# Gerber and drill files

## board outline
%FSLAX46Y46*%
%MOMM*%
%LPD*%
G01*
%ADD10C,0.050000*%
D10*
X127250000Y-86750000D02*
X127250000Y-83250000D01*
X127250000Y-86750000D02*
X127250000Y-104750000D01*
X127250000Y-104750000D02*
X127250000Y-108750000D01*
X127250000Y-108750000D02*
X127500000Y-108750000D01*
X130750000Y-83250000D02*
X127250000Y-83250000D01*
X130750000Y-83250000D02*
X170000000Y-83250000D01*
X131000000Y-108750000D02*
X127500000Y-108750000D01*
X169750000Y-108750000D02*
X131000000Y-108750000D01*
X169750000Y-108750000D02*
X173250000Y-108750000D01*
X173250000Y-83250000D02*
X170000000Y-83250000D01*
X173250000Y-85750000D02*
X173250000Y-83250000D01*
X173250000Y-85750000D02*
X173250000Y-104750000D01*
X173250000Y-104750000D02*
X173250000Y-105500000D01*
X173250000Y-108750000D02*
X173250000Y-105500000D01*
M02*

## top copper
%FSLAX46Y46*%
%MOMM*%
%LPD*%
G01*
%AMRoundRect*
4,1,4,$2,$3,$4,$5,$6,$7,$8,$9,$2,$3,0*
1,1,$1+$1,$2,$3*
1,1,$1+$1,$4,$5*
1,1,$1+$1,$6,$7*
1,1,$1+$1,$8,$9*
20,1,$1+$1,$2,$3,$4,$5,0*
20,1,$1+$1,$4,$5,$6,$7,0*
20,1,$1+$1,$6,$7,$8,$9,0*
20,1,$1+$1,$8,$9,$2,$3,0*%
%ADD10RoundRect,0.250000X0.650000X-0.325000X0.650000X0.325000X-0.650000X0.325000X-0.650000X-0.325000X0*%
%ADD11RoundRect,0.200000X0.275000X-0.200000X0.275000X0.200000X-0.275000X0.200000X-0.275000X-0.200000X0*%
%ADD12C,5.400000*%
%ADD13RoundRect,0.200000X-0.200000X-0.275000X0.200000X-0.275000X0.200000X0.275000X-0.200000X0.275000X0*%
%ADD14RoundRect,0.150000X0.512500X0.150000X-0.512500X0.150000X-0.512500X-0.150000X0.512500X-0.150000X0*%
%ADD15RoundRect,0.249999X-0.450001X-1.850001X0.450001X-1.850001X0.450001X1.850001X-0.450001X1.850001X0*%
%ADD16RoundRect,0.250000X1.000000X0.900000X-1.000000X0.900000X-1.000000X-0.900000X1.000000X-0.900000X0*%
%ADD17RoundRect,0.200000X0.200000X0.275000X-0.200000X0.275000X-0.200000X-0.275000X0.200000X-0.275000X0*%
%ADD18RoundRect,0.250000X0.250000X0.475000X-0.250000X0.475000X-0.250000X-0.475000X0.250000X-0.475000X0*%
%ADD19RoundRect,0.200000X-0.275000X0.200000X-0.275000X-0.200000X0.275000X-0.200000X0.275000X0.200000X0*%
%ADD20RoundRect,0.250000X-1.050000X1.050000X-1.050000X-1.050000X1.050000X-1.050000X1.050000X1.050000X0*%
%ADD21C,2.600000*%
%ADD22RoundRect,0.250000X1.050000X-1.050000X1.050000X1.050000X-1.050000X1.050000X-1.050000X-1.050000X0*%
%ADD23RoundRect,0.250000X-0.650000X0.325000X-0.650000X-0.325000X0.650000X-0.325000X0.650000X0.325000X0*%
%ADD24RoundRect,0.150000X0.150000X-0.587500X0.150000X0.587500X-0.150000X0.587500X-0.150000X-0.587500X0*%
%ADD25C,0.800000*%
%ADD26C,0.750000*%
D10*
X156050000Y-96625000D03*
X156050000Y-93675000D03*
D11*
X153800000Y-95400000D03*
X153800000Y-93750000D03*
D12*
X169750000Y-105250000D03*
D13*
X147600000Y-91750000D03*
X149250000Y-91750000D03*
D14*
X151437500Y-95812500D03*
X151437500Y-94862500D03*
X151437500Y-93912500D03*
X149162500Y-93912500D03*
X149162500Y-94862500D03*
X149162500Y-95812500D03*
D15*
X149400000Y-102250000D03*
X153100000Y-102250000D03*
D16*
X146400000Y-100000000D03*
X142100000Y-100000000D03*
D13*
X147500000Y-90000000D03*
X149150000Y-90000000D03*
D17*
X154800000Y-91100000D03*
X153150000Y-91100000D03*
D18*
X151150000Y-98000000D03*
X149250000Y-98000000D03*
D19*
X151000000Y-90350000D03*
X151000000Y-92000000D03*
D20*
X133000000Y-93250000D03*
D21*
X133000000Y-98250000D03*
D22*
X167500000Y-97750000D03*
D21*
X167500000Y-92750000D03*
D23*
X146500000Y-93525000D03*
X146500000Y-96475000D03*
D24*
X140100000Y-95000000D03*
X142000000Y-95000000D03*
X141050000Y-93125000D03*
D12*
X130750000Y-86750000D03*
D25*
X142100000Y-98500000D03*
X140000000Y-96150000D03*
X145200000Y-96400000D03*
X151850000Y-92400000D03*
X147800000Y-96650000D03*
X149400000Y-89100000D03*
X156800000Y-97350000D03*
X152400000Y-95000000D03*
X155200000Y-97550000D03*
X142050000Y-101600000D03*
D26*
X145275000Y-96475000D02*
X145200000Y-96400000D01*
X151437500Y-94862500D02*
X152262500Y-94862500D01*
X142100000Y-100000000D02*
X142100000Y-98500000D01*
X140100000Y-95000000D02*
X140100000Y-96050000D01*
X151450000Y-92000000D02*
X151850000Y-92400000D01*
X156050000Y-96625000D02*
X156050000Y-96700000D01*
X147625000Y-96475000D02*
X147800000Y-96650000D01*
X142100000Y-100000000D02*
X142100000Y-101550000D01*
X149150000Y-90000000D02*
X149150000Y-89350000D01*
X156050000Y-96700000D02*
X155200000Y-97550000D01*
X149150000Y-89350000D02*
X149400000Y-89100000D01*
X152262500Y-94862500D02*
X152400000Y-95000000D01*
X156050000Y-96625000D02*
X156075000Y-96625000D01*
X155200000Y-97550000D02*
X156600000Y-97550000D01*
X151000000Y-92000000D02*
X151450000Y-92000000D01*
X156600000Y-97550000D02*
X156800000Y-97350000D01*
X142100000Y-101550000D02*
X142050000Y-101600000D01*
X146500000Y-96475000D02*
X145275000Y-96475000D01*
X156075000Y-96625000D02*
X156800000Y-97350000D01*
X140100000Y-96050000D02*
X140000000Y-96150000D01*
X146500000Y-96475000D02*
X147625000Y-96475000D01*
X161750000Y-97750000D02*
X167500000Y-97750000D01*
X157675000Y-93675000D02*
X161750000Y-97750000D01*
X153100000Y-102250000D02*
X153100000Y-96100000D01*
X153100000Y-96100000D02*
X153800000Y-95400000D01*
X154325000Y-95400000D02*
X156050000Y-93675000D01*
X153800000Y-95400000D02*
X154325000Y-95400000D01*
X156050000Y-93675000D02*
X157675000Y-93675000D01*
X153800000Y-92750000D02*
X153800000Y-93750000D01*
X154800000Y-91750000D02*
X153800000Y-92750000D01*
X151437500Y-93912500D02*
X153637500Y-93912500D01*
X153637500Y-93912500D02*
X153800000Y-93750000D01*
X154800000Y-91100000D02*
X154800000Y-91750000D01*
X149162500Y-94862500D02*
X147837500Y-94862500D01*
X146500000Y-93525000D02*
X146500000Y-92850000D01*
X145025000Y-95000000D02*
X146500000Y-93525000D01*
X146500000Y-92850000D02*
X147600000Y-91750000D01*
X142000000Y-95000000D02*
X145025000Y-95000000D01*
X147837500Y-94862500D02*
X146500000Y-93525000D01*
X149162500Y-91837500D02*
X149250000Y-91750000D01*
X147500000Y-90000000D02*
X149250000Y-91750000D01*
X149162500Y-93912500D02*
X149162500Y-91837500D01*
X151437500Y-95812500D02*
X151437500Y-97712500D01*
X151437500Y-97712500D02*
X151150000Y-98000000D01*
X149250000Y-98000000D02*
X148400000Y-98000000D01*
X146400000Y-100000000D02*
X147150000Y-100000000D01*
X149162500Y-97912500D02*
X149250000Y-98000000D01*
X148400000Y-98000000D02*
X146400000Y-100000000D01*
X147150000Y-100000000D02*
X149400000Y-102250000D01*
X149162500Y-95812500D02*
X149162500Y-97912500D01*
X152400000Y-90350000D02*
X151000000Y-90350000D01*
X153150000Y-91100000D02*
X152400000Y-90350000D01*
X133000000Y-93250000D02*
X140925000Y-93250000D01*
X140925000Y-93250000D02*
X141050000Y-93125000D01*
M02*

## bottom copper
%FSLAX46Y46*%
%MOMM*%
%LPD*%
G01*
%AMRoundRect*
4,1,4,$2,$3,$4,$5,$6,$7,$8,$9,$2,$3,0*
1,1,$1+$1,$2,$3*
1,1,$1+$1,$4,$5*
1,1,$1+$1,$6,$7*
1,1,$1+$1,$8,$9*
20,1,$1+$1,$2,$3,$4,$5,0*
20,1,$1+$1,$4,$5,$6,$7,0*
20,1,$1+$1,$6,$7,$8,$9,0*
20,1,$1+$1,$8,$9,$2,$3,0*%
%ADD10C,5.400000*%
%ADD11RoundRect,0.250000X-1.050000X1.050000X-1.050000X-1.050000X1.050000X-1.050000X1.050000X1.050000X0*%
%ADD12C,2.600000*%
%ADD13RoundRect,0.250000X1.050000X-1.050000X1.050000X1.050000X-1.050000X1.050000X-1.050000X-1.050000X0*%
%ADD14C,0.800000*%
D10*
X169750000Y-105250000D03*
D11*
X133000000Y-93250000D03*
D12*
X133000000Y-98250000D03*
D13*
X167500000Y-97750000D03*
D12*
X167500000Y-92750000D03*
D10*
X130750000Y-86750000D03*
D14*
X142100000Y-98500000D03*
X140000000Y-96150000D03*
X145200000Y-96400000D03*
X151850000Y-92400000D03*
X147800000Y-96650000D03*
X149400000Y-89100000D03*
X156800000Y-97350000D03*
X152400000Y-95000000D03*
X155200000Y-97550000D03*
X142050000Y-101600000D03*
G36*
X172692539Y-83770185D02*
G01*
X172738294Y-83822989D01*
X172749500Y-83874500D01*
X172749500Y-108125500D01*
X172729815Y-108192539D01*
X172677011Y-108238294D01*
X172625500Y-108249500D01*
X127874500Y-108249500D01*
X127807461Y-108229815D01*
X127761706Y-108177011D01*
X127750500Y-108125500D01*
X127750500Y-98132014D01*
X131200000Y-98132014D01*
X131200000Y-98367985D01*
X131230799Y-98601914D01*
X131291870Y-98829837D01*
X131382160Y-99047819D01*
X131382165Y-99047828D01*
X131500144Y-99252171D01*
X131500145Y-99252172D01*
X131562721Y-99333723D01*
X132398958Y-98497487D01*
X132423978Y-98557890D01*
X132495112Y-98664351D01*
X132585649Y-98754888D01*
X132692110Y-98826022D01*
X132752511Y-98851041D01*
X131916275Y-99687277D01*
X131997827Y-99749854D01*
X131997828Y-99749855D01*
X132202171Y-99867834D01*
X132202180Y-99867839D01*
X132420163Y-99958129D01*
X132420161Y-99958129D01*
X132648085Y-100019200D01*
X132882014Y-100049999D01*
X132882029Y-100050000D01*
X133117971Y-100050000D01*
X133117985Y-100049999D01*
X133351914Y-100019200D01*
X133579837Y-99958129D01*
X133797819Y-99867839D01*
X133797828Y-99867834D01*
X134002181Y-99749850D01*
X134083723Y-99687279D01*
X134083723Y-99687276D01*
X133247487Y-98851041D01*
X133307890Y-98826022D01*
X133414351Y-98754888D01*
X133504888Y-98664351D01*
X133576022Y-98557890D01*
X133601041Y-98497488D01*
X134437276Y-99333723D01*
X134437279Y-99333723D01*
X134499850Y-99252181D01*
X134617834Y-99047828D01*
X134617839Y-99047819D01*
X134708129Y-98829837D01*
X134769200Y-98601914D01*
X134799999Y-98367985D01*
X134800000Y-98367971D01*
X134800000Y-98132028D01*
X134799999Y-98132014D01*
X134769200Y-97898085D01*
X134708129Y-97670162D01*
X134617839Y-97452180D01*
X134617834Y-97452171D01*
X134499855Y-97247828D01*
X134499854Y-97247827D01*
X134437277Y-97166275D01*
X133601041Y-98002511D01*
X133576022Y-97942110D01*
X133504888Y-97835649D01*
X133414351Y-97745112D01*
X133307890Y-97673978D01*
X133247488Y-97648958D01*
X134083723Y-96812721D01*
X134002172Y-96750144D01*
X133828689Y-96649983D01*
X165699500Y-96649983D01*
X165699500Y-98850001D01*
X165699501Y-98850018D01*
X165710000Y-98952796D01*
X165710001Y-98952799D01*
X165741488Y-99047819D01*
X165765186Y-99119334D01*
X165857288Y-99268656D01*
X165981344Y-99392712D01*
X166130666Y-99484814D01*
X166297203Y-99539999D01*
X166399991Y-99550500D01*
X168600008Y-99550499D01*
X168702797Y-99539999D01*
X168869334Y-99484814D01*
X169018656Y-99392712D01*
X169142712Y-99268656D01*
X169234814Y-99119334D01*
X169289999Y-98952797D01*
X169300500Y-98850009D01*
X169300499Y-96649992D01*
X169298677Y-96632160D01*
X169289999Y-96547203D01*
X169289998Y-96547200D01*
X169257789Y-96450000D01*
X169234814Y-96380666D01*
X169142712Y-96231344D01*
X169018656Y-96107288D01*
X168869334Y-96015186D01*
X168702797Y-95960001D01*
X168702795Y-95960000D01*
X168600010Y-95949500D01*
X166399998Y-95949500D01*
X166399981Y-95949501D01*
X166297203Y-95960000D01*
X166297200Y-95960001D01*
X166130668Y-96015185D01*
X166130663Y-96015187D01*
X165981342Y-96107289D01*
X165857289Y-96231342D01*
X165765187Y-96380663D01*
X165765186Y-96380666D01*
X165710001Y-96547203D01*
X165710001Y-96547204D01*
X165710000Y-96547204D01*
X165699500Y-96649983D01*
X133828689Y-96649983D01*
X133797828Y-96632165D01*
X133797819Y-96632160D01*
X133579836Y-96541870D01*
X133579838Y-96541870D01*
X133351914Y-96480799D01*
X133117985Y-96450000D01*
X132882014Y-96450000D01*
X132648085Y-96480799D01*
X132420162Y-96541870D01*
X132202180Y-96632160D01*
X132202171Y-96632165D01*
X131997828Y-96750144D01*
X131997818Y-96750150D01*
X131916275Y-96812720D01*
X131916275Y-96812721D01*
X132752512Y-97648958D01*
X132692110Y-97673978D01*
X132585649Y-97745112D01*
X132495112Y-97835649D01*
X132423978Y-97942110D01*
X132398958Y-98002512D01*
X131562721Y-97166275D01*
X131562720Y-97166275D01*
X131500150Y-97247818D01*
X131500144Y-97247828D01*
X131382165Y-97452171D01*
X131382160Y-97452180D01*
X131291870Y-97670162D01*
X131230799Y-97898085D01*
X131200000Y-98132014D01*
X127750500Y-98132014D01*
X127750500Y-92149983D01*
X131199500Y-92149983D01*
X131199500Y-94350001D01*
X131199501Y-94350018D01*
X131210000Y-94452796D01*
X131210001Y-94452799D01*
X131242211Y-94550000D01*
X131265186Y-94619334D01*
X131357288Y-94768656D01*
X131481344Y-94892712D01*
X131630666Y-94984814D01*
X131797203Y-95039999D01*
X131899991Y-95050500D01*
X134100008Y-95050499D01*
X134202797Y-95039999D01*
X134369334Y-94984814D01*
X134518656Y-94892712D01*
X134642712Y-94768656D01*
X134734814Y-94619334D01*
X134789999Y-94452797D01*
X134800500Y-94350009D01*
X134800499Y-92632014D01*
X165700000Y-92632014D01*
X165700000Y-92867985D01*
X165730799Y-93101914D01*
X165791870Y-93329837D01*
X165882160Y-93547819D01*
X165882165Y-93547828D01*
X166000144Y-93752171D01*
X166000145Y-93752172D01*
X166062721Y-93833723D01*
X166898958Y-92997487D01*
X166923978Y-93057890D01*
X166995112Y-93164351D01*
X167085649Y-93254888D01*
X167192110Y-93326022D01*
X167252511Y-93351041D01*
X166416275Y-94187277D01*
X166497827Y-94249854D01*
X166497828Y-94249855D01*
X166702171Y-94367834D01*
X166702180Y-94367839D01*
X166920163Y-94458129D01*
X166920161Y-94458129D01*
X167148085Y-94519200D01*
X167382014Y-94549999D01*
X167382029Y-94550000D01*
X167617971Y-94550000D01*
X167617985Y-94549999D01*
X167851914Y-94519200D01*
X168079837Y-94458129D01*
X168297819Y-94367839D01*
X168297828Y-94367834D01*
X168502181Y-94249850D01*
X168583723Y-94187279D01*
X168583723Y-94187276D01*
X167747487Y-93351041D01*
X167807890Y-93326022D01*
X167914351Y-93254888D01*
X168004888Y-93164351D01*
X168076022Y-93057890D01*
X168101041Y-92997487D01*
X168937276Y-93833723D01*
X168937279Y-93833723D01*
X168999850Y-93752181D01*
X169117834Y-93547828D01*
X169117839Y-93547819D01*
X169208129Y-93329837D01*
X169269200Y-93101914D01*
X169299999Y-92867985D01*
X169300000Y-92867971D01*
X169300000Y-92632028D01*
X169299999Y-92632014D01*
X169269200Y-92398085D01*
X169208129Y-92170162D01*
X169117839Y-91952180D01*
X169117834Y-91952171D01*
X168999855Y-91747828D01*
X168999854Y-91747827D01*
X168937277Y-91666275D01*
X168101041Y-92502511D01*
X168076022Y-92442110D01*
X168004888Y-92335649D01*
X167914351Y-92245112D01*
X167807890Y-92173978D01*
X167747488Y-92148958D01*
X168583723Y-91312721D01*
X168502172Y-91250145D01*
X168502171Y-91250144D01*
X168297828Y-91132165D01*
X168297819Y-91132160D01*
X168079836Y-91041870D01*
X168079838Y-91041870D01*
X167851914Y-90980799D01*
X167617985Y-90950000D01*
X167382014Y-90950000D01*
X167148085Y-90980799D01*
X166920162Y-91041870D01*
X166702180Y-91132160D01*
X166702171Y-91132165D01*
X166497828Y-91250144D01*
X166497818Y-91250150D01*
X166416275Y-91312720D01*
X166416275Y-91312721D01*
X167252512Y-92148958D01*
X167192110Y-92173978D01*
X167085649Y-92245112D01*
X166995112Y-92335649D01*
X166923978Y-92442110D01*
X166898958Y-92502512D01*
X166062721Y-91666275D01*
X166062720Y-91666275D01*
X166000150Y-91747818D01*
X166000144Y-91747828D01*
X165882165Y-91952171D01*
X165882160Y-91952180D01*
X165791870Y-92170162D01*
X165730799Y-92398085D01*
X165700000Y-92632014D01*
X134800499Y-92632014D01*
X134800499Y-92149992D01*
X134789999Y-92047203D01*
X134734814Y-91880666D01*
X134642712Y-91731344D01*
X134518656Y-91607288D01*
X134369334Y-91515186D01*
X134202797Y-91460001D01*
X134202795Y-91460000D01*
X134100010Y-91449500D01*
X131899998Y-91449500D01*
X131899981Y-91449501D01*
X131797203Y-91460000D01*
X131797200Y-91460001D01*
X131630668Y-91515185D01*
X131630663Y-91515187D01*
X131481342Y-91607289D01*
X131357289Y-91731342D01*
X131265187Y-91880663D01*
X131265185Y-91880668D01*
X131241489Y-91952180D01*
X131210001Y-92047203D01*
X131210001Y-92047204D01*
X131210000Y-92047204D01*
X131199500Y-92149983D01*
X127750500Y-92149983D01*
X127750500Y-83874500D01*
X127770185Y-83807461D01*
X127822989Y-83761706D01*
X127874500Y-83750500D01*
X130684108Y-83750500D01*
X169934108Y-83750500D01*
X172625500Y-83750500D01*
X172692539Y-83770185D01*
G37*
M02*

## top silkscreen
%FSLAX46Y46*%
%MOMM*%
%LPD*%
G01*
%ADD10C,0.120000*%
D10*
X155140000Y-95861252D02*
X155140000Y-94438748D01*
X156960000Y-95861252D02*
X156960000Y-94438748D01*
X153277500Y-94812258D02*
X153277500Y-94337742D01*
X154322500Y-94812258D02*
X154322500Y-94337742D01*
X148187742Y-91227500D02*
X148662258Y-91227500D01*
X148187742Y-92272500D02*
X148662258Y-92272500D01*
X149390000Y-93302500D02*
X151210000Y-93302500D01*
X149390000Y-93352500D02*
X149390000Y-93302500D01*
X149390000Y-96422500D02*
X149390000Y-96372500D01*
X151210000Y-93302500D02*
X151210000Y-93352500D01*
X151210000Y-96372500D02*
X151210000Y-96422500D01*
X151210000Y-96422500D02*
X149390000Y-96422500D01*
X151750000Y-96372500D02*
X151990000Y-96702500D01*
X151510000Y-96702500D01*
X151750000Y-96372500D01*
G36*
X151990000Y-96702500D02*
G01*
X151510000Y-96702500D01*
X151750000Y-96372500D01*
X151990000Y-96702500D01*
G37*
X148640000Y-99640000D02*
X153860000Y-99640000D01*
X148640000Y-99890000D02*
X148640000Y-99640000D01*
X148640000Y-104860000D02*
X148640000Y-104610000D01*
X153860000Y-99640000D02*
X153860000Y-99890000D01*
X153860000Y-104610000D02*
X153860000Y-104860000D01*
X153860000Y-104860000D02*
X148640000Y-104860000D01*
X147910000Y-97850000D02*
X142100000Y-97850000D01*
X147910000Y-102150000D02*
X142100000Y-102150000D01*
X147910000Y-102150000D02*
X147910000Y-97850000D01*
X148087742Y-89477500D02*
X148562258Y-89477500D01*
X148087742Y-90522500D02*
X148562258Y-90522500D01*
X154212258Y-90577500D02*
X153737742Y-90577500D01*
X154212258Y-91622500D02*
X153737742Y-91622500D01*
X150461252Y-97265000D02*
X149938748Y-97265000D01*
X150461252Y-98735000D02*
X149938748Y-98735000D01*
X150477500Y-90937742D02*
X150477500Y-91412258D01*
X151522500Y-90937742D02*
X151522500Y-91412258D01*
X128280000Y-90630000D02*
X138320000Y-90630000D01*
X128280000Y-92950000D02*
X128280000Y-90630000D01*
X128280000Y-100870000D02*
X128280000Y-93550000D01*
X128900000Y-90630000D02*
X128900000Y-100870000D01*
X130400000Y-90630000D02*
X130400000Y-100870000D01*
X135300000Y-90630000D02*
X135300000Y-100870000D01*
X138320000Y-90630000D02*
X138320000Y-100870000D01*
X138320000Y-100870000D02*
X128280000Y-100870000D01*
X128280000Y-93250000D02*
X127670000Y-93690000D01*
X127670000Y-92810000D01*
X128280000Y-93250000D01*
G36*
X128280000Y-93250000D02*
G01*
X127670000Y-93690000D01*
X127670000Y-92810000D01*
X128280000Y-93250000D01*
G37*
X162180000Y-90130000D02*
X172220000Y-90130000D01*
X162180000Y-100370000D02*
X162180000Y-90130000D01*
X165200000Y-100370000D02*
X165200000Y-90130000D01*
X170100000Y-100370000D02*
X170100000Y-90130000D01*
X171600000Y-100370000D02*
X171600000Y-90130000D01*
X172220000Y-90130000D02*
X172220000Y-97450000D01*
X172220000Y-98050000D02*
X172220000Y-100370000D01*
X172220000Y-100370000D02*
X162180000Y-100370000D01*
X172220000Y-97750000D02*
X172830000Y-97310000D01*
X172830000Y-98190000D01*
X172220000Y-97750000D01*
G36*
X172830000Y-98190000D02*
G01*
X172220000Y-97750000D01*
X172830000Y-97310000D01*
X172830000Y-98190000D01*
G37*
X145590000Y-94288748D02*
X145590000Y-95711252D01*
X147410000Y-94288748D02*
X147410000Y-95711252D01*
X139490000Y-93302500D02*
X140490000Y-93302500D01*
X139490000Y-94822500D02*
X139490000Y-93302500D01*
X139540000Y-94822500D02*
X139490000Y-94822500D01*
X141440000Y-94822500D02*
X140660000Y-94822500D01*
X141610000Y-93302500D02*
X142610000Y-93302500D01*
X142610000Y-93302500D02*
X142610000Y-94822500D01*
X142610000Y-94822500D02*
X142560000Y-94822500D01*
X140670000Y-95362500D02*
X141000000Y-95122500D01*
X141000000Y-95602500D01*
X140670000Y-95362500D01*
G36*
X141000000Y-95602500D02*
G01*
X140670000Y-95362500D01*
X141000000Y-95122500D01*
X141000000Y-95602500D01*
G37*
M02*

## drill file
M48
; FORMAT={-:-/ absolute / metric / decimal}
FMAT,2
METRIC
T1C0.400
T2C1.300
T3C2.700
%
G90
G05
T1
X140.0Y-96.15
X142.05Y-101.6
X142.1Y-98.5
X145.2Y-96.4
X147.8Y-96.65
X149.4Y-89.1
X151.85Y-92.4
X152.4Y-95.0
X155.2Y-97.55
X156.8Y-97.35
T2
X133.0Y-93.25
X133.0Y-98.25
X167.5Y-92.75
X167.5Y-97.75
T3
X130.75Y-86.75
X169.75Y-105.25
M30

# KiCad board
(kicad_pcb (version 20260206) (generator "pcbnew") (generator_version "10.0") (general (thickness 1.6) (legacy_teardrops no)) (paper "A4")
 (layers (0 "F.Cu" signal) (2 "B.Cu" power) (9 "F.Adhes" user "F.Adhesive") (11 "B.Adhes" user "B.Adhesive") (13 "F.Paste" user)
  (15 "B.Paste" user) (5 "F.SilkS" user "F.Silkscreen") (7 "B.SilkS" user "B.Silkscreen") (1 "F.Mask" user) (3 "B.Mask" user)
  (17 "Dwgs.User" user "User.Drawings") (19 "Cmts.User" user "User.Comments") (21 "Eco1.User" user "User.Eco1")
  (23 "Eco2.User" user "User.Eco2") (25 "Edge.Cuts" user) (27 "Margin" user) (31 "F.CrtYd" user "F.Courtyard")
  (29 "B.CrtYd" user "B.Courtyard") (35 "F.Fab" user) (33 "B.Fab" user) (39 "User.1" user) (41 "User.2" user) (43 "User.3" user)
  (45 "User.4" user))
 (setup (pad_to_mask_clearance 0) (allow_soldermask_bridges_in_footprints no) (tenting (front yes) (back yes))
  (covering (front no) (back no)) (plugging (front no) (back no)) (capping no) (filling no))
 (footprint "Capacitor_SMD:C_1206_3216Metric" (layer "F.Cu") (at 156.05 95.15 90)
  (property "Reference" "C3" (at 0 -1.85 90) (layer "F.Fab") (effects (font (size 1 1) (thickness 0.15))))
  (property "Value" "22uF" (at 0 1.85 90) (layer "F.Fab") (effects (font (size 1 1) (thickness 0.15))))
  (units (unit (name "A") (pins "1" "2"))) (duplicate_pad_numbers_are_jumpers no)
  (fp_line (start -0.711252 -0.91) (end 0.711252 -0.91) (stroke (width 0.12) (type solid)) (layer "F.SilkS"))
  (fp_line (start -0.711252 0.91) (end 0.711252 0.91) (stroke (width 0.12) (type solid)) (layer "F.SilkS"))
  (pad "1" smd roundrect (at -1.475 0 90) (size 1.15 1.8) (layers "F.Cu" "F.Mask" "F.Paste") (roundrect_rratio 0.217391) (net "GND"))
  (pad "2" smd roundrect (at 1.475 0 90) (size 1.15 1.8) (layers "F.Cu" "F.Mask" "F.Paste") (roundrect_rratio 0.217391) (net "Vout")))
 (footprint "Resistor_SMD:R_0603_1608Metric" (layer "F.Cu") (at 153.8 94.575 90)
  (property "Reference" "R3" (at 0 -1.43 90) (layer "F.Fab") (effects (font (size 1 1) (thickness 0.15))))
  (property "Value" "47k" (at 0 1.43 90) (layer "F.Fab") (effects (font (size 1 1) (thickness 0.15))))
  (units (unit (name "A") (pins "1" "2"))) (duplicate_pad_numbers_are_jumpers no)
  (fp_line (start -0.237258 -0.5225) (end 0.237258 -0.5225) (stroke (width 0.12) (type solid)) (layer "F.SilkS"))
  (fp_line (start -0.237258 0.5225) (end 0.237258 0.5225) (stroke (width 0.12) (type solid)) (layer "F.SilkS"))
  (pad "1" smd roundrect (at -0.825 0 90) (size 0.8 0.95) (layers "F.Cu" "F.Mask" "F.Paste") (roundrect_rratio 0.25) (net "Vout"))
  (pad "2" smd roundrect (at 0.825 0 90) (size 0.8 0.95) (layers "F.Cu" "F.Mask" "F.Paste") (roundrect_rratio 0.25) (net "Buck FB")))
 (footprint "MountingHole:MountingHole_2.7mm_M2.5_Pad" (layer "F.Cu") (at 169.75 105.25)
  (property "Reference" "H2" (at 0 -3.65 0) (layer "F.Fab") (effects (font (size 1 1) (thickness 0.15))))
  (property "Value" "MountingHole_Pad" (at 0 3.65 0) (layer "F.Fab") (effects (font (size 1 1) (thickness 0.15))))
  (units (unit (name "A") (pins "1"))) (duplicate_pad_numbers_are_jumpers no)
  (pad "1" thru_hole circle (at 0 0) (size 5.4 5.4) (drill 2.7) (layers "*.Cu" "*.Mask") (remove_unused_layers no) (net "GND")
   (zone_connect 2)))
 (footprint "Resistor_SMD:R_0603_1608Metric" (layer "F.Cu") (at 148.425 91.75)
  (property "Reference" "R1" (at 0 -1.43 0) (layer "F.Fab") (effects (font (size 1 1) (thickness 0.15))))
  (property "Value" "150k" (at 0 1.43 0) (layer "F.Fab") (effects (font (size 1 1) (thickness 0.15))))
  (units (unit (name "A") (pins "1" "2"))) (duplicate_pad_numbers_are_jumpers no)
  (fp_line (start -0.237258 -0.5225) (end 0.237258 -0.5225) (stroke (width 0.12) (type solid)) (layer "F.SilkS"))
  (fp_line (start -0.237258 0.5225) (end 0.237258 0.5225) (stroke (width 0.12) (type solid)) (layer "F.SilkS"))
  (pad "1" smd roundrect (at -0.825 0) (size 0.8 0.95) (layers "F.Cu" "F.Mask" "F.Paste") (roundrect_rratio 0.25) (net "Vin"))
  (pad "2" smd roundrect (at 0.825 0) (size 0.8 0.95) (layers "F.Cu" "F.Mask" "F.Paste") (roundrect_rratio 0.25) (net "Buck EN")))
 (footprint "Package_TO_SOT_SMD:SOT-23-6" (layer "F.Cu") (at 150.3 94.8625 180)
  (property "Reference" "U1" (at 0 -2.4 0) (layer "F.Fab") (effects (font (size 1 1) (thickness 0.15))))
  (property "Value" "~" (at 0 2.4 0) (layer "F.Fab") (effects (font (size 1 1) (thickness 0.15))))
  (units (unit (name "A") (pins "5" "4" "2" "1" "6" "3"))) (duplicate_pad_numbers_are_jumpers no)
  (fp_line (start 0.91 1.56) (end -0.91 1.56) (stroke (width 0.12) (type solid)) (layer "F.SilkS"))
  (fp_line (start 0.91 1.51) (end 0.91 1.56) (stroke (width 0.12) (type solid)) (layer "F.SilkS"))
  (fp_line (start 0.91 -1.56) (end 0.91 -1.51) (stroke (width 0.12) (type solid)) (layer "F.SilkS"))
  (fp_line (start -0.91 1.56) (end -0.91 1.51) (stroke (width 0.12) (type solid)) (layer "F.SilkS"))
  (fp_line (start -0.91 -1.51) (end -0.91 -1.56) (stroke (width 0.12) (type solid)) (layer "F.SilkS"))
  (fp_line (start -0.91 -1.56) (end 0.91 -1.56) (stroke (width 0.12) (type solid)) (layer "F.SilkS"))
  (fp_poly (pts (xy -1.45 -1.51) (xy -1.69 -1.84) (xy -1.21 -1.84)) (stroke (width 0.12) (type solid)) (fill yes) (layer "F.SilkS"))
  (pad "1" smd roundrect (at -1.1375 -0.95 180) (size 1.325 0.6) (layers "F.Cu" "F.Mask" "F.Paste") (roundrect_rratio 0.25) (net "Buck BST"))
  (pad "2" smd roundrect (at -1.1375 0 180) (size 1.325 0.6) (layers "F.Cu" "F.Mask" "F.Paste") (roundrect_rratio 0.25) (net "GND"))
  (pad "3" smd roundrect (at -1.1375 0.95 180) (size 1.325 0.6) (layers "F.Cu" "F.Mask" "F.Paste") (roundrect_rratio 0.25) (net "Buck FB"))
  (pad "4" smd roundrect (at 1.1375 0.95 180) (size 1.325 0.6) (layers "F.Cu" "F.Mask" "F.Paste") (roundrect_rratio 0.25) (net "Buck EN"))
  (pad "5" smd roundrect (at 1.1375 0 180) (size 1.325 0.6) (layers "F.Cu" "F.Mask" "F.Paste") (roundrect_rratio 0.25) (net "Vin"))
  (pad "6" smd roundrect (at 1.1375 -0.95 180) (size 1.325 0.6) (layers "F.Cu" "F.Mask" "F.Paste") (roundrect_rratio 0.25) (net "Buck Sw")))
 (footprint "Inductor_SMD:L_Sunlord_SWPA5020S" (layer "F.Cu") (at 151.25 102.25)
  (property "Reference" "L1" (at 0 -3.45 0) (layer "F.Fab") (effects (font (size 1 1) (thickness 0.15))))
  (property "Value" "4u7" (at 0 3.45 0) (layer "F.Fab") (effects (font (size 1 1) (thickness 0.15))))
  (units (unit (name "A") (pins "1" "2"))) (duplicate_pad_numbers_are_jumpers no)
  (fp_line (start -2.61 -2.61) (end 2.61 -2.61) (stroke (width 0.12) (type solid)) (layer "F.SilkS"))
  (fp_line (start -2.61 -2.36) (end -2.61 -2.61) (stroke (width 0.12) (type solid)) (layer "F.SilkS"))
  (fp_line (start -2.61 2.61) (end -2.61 2.36) (stroke (width 0.12) (type solid)) (layer "F.SilkS"))
  (fp_line (start 2.61 -2.61) (end 2.61 -2.36) (stroke (width 0.12) (type solid)) (layer "F.SilkS"))
  (fp_line (start 2.61 2.36) (end 2.61 2.61) (stroke (width 0.12) (type solid)) (layer "F.SilkS"))
  (fp_line (start 2.61 2.61) (end -2.61 2.61) (stroke (width 0.12) (type solid)) (layer "F.SilkS"))
  (pad "1" smd roundrect (at -1.85 0) (size 1.4 4.2) (layers "F.Cu" "F.Mask" "F.Paste") (roundrect_rratio 0.178571) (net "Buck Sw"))
  (pad "2" smd roundrect (at 1.85 0) (size 1.4 4.2) (layers "F.Cu" "F.Mask" "F.Paste") (roundrect_rratio 0.178571) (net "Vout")))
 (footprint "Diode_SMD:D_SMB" (layer "F.Cu") (at 144.25 100 180)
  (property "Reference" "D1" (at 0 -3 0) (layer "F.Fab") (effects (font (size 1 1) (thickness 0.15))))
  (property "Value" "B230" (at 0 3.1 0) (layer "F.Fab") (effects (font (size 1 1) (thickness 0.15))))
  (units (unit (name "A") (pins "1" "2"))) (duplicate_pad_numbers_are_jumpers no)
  (fp_line (start -3.66 2.15) (end 2.15 2.15) (stroke (width 0.12) (type solid)) (layer "F.SilkS"))
  (fp_line (start -3.66 -2.15) (end 2.15 -2.15) (stroke (width 0.12) (type solid)) (layer "F.SilkS"))
  (fp_line (start -3.66 -2.15) (end -3.66 2.15) (stroke (width 0.12) (type solid)) (layer "F.SilkS"))
  (pad "1" smd roundrect (at -2.15 0 180) (size 2.5 2.3) (layers "F.Cu" "F.Mask" "F.Paste") (roundrect_rratio 0.1086956522) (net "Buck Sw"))
  (pad "2" smd roundrect (at 2.15 0 180) (size 2.5 2.3) (layers "F.Cu" "F.Mask" "F.Paste") (roundrect_rratio 0.1086956522) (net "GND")))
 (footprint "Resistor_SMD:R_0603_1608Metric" (layer "F.Cu") (at 148.325 90)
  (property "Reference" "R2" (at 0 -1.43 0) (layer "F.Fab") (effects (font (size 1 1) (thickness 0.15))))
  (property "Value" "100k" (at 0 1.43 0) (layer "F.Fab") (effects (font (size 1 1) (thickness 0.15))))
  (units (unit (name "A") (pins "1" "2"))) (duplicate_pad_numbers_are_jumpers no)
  (fp_line (start -0.237258 -0.5225) (end 0.237258 -0.5225) (stroke (width 0.12) (type solid)) (layer "F.SilkS"))
  (fp_line (start -0.237258 0.5225) (end 0.237258 0.5225) (stroke (width 0.12) (type solid)) (layer "F.SilkS"))
  (pad "1" smd roundrect (at -0.825 0) (size 0.8 0.95) (layers "F.Cu" "F.Mask" "F.Paste") (roundrect_rratio 0.25) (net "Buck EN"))
  (pad "2" smd roundrect (at 0.825 0) (size 0.8 0.95) (layers "F.Cu" "F.Mask" "F.Paste") (roundrect_rratio 0.25) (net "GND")))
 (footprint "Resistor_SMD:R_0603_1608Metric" (layer "F.Cu") (at 153.975 91.1 180)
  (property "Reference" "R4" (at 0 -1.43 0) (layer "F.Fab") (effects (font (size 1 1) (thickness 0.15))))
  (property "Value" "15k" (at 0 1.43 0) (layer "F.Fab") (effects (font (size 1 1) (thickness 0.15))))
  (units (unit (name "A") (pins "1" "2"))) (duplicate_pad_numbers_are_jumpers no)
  (fp_line (start -0.237258 0.5225) (end 0.237258 0.5225) (stroke (width 0.12) (type solid)) (layer "F.SilkS"))
  (fp_line (start -0.237258 -0.5225) (end 0.237258 -0.5225) (stroke (width 0.12) (type solid)) (layer "F.SilkS"))
  (pad "1" smd roundrect (at -0.825 0 180) (size 0.8 0.95) (layers "F.Cu" "F.Mask" "F.Paste") (roundrect_rratio 0.25) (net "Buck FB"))
  (pad "2" smd roundrect (at 0.825 0 180) (size 0.8 0.95) (layers "F.Cu" "F.Mask" "F.Paste") (roundrect_rratio 0.25) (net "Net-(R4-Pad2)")))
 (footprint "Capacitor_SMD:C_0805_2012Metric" (layer "F.Cu") (at 150.2 98 180)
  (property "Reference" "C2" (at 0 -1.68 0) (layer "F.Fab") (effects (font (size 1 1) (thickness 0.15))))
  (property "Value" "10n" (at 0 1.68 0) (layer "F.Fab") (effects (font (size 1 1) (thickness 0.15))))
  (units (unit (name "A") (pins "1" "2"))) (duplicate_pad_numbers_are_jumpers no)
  (fp_line (start -0.261252 0.735) (end 0.261252 0.735) (stroke (width 0.12) (type solid)) (layer "F.SilkS"))
  (fp_line (start -0.261252 -0.735) (end 0.261252 -0.735) (stroke (width 0.12) (type solid)) (layer "F.SilkS"))
  (pad "1" smd roundrect (at -0.95 0 180) (size 1 1.45) (layers "F.Cu" "F.Mask" "F.Paste") (roundrect_rratio 0.25) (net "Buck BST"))
  (pad "2" smd roundrect (at 0.95 0 180) (size 1 1.45) (layers "F.Cu" "F.Mask" "F.Paste") (roundrect_rratio 0.25) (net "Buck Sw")))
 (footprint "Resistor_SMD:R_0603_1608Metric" (layer "F.Cu") (at 151 91.175 -90)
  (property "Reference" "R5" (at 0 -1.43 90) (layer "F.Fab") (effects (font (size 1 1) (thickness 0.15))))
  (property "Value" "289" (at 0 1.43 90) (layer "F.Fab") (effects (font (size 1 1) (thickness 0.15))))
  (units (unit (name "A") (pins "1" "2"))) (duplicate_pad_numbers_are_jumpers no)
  (fp_line (start -0.237258 0.5225) (end 0.237258 0.5225) (stroke (width 0.12) (type solid)) (layer "F.SilkS"))
  (fp_line (start -0.237258 -0.5225) (end 0.237258 -0.5225) (stroke (width 0.12) (type solid)) (layer "F.SilkS"))
  (pad "1" smd roundrect (at -0.825 0 270) (size 0.8 0.95) (layers "F.Cu" "F.Mask" "F.Paste") (roundrect_rratio 0.25) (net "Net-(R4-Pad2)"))
  (pad "2" smd roundrect (at 0.825 0 270) (size 0.8 0.95) (layers "F.Cu" "F.Mask" "F.Paste") (roundrect_rratio 0.25) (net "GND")))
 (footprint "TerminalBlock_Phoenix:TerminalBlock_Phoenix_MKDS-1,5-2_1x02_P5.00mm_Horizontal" (layer "F.Cu") (at 133 93.25 -90)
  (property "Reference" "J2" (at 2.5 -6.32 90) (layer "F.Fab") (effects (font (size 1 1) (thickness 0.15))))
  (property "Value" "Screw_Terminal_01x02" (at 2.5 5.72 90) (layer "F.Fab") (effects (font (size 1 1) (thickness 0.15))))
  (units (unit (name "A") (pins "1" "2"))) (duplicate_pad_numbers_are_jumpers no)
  (fp_line (start -2.62 4.72) (end -2.62 -5.32) (stroke (width 0.12) (type solid)) (layer "F.SilkS"))
  (fp_line (start -0.3 4.72) (end -2.62 4.72) (stroke (width 0.12) (type solid)) (layer "F.SilkS"))
  (fp_line (start 7.62 4.72) (end 0.3 4.72) (stroke (width 0.12) (type solid)) (layer "F.SilkS"))
  (fp_line (start -2.62 4.1) (end 7.62 4.1) (stroke (width 0.12) (type solid)) (layer "F.SilkS"))
  (fp_line (start -2.62 2.6) (end 7.62 2.6) (stroke (width 0.12) (type solid)) (layer "F.SilkS"))
  (fp_line (start -2.62 -2.3) (end 7.62 -2.3) (stroke (width 0.12) (type solid)) (layer "F.SilkS"))
  (fp_line (start -2.62 -5.32) (end 7.62 -5.32) (stroke (width 0.12) (type solid)) (layer "F.SilkS"))
  (fp_line (start 7.62 -5.32) (end 7.62 4.72) (stroke (width 0.12) (type solid)) (layer "F.SilkS"))
  (fp_poly (pts (xy 0 4.72) (xy 0.44 5.33) (xy -0.44 5.33)) (stroke (width 0.12) (type solid)) (fill yes) (layer "F.SilkS"))
  (pad "1" thru_hole roundrect (at 0 0 270) (size 2.6 2.6) (drill 1.3) (layers "*.Cu" "*.Mask") (remove_unused_layers no)
   (roundrect_rratio 0.096154) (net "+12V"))
  (pad "2" thru_hole circle (at 5 0 270) (size 2.6 2.6) (drill 1.3) (layers "*.Cu" "*.Mask") (remove_unused_layers no) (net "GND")))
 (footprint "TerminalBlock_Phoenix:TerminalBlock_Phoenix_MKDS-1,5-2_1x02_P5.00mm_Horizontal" (layer "F.Cu") (at 167.5 97.75 90)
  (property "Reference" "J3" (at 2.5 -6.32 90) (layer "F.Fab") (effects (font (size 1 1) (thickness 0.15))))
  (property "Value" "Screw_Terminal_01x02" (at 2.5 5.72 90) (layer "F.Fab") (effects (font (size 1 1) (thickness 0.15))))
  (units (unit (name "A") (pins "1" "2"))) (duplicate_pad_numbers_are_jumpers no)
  (fp_line (start 7.62 -5.32) (end 7.62 4.72) (stroke (width 0.12) (type solid)) (layer "F.SilkS"))
  (fp_line (start -2.62 -5.32) (end 7.62 -5.32) (stroke (width 0.12) (type solid)) (layer "F.SilkS"))
  (fp_line (start -2.62 -2.3) (end 7.62 -2.3) (stroke (width 0.12) (type solid)) (layer "F.SilkS"))
  (fp_line (start -2.62 2.6) (end 7.62 2.6) (stroke (width 0.12) (type solid)) (layer "F.SilkS"))
  (fp_line (start -2.62 4.1) (end 7.62 4.1) (stroke (width 0.12) (type solid)) (layer "F.SilkS"))
  (fp_line (start 7.62 4.72) (end 0.3 4.72) (stroke (width 0.12) (type solid)) (layer "F.SilkS"))
  (fp_line (start -0.3 4.72) (end -2.62 4.72) (stroke (width 0.12) (type solid)) (layer "F.SilkS"))
  (fp_line (start -2.62 4.72) (end -2.62 -5.32) (stroke (width 0.12) (type solid)) (layer "F.SilkS"))
  (fp_poly (pts (xy 0 4.72) (xy 0.44 5.33) (xy -0.44 5.33)) (stroke (width 0.12) (type solid)) (fill yes) (layer "F.SilkS"))
  (pad "1" thru_hole roundrect (at 0 0 90) (size 2.6 2.6) (drill 1.3) (layers "*.Cu" "*.Mask") (remove_unused_layers no)
   (roundrect_rratio 0.096154) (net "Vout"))
  (pad "2" thru_hole circle (at 5 0 90) (size 2.6 2.6) (drill 1.3) (layers "*.Cu" "*.Mask") (remove_unused_layers no) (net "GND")))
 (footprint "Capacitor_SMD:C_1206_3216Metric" (layer "F.Cu") (at 146.5 95 -90)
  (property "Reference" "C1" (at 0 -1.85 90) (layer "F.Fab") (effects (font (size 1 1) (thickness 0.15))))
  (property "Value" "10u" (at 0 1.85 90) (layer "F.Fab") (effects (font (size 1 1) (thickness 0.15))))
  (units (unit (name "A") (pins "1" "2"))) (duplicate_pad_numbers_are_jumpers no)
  (fp_line (start -0.711252 0.91) (end 0.711252 0.91) (stroke (width 0.12) (type solid)) (layer "F.SilkS"))
  (fp_line (start -0.711252 -0.91) (end 0.711252 -0.91) (stroke (width 0.12) (type solid)) (layer "F.SilkS"))
  (pad "1" smd roundrect (at -1.475 0 270) (size 1.15 1.8) (layers "F.Cu" "F.Mask" "F.Paste") (roundrect_rratio 0.217391) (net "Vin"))
  (pad "2" smd roundrect (at 1.475 0 270) (size 1.15 1.8) (layers "F.Cu" "F.Mask" "F.Paste") (roundrect_rratio 0.217391) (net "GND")))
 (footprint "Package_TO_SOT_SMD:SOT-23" (layer "F.Cu") (at 141.05 94.0625 90)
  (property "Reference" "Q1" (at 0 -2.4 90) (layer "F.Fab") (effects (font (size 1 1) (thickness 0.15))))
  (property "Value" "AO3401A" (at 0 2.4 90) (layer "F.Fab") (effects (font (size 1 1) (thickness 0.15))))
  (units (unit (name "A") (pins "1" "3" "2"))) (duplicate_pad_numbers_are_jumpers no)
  (fp_line (start 0.76 -1.56) (end 0.76 -0.56) (stroke (width 0.12) (type solid)) (layer "F.SilkS"))
  (fp_line (start -0.76 -1.56) (end 0.76 -1.56) (stroke (width 0.12) (type solid)) (layer "F.SilkS"))
  (fp_line (start -0.76 -1.51) (end -0.76 -1.56) (stroke (width 0.12) (type solid)) (layer "F.SilkS"))
  (fp_line (start -0.76 0.39) (end -0.76 -0.39) (stroke (width 0.12) (type solid)) (layer "F.SilkS"))
  (fp_line (start 0.76 0.56) (end 0.76 1.56) (stroke (width 0.12) (type solid)) (layer "F.SilkS"))
  (fp_line (start 0.76 1.56) (end -0.76 1.56) (stroke (width 0.12) (type solid)) (layer "F.SilkS"))
  (fp_line (start -0.76 1.56) (end -0.76 1.51) (stroke (width 0.12) (type solid)) (layer "F.SilkS"))
  (fp_poly (pts (xy -1.3 -0.38) (xy -1.06 -0.05) (xy -1.54 -0.05)) (stroke (width 0.12) (type solid)) (fill yes) (layer "F.SilkS"))
  (pad "1" smd roundrect (at -0.9375 -0.95 90) (size 1.475 0.6) (layers "F.Cu" "F.Mask" "F.Paste") (roundrect_rratio 0.25) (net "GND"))
  (pad "2" smd roundrect (at -0.9375 0.95 90) (size 1.475 0.6) (layers "F.Cu" "F.Mask" "F.Paste") (roundrect_rratio 0.25) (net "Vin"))
  (pad "3" smd roundrect (at 0.9375 0 90) (size 1.475 0.6) (layers "F.Cu" "F.Mask" "F.Paste") (roundrect_rratio 0.25) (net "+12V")))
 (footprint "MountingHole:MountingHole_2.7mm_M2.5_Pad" (layer "F.Cu") (at 130.75 86.75)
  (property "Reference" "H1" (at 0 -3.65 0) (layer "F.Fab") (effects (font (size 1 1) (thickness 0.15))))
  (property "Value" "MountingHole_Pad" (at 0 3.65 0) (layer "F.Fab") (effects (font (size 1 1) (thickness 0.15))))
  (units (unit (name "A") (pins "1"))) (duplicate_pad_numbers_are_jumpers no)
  (pad "1" thru_hole circle (at 0 0) (size 5.4 5.4) (drill 2.7) (layers "*.Cu" "*.Mask") (remove_unused_layers no) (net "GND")
   (zone_connect 2)))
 (gr_line (start 127.25 86.75) (end 127.25 83.25) (stroke (width 0.05) (type default)) (layer "Edge.Cuts"))
 (gr_line (start 127.25 86.75) (end 127.25 104.75) (stroke (width 0.05) (type default)) (layer "Edge.Cuts"))
 (gr_line (start 127.25 104.75) (end 127.25 108.75) (stroke (width 0.05) (type default)) (layer "Edge.Cuts"))
 (gr_line (start 127.25 108.75) (end 127.5 108.75) (stroke (width 0.05) (type default)) (layer "Edge.Cuts"))
 (gr_line (start 130.75 83.25) (end 127.25 83.25) (stroke (width 0.05) (type default)) (layer "Edge.Cuts"))
 (gr_line (start 130.75 83.25) (end 170 83.25) (stroke (width 0.05) (type default)) (layer "Edge.Cuts"))
 (gr_line (start 131 108.75) (end 127.5 108.75) (stroke (width 0.05) (type default)) (layer "Edge.Cuts"))
 (gr_line (start 169.75 108.75) (end 131 108.75) (stroke (width 0.05) (type default)) (layer "Edge.Cuts"))
 (gr_line (start 169.75 108.75) (end 173.25 108.75) (stroke (width 0.05) (type default)) (layer "Edge.Cuts"))
 (gr_line (start 173.25 83.25) (end 170 83.25) (stroke (width 0.05) (type default)) (layer "Edge.Cuts"))
 (gr_line (start 173.25 85.75) (end 173.25 83.25) (stroke (width 0.05) (type default)) (layer "Edge.Cuts"))
 (gr_line (start 173.25 85.75) (end 173.25 104.75) (stroke (width 0.05) (type default)) (layer "Edge.Cuts"))
 (gr_line (start 173.25 104.75) (end 173.25 105.5) (stroke (width 0.05) (type default)) (layer "Edge.Cuts"))
 (gr_line (start 173.25 108.75) (end 173.25 105.5) (stroke (width 0.05) (type default)) (layer "Edge.Cuts"))
 (segment (start 145.275 96.475) (end 145.2 96.4) (width 0.75) (layer "F.Cu") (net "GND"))
 (segment (start 151.4375 94.8625) (end 152.2625 94.8625) (width 0.75) (layer "F.Cu") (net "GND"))
 (segment (start 142.1 100) (end 142.1 98.5) (width 0.75) (layer "F.Cu") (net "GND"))
 (segment (start 140.1 95) (end 140.1 96.05) (width 0.75) (layer "F.Cu") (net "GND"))
 (segment (start 151.45 92) (end 151.85 92.4) (width 0.75) (layer "F.Cu") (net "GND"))
 (segment (start 156.05 96.625) (end 156.05 96.7) (width 0.75) (layer "F.Cu") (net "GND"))
 (segment (start 147.625 96.475) (end 147.8 96.65) (width 0.75) (layer "F.Cu") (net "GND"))
 (segment (start 142.1 100) (end 142.1 101.55) (width 0.75) (layer "F.Cu") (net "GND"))
 (segment (start 149.15 90) (end 149.15 89.35) (width 0.75) (layer "F.Cu") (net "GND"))
 (segment (start 156.05 96.7) (end 155.2 97.55) (width 0.75) (layer "F.Cu") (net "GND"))
 (segment (start 149.15 89.35) (end 149.4 89.1) (width 0.75) (layer "F.Cu") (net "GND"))
 (segment (start 152.2625 94.8625) (end 152.4 95) (width 0.75) (layer "F.Cu") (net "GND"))
 (segment (start 156.05 96.625) (end 156.075 96.625) (width 0.75) (layer "F.Cu") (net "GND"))
 (segment (start 155.2 97.55) (end 156.6 97.55) (width 0.75) (layer "F.Cu") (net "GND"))
 (segment (start 151 92) (end 151.45 92) (width 0.75) (layer "F.Cu") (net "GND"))
 (segment (start 156.6 97.55) (end 156.8 97.35) (width 0.75) (layer "F.Cu") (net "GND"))
 (segment (start 142.1 101.55) (end 142.05 101.6) (width 0.75) (layer "F.Cu") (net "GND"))
 (segment (start 146.5 96.475) (end 145.275 96.475) (width 0.75) (layer "F.Cu") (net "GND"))
 (segment (start 156.075 96.625) (end 156.8 97.35) (width 0.75) (layer "F.Cu") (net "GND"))
 (segment (start 140.1 96.05) (end 140 96.15) (width 0.75) (layer "F.Cu") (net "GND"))
 (segment (start 146.5 96.475) (end 147.625 96.475) (width 0.75) (layer "F.Cu") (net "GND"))
 (via (at 142.1 98.5) (size 0.8) (drill 0.4) (layers "F.Cu" "B.Cu") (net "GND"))
 (via (at 140 96.15) (size 0.8) (drill 0.4) (layers "F.Cu" "B.Cu") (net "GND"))
 (via (at 145.2 96.4) (size 0.8) (drill 0.4) (layers "F.Cu" "B.Cu") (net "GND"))
 (via (at 151.85 92.4) (size 0.8) (drill 0.4) (layers "F.Cu" "B.Cu") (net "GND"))
 (via (at 147.8 96.65) (size 0.8) (drill 0.4) (layers "F.Cu" "B.Cu") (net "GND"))
 (via (at 149.4 89.1) (size 0.8) (drill 0.4) (layers "F.Cu" "B.Cu") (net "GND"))
 (via (at 156.8 97.35) (size 0.8) (drill 0.4) (layers "F.Cu" "B.Cu") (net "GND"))
 (via (at 152.4 95) (size 0.8) (drill 0.4) (layers "F.Cu" "B.Cu") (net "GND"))
 (via (at 155.2 97.55) (size 0.8) (drill 0.4) (layers "F.Cu" "B.Cu") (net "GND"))
 (via (at 142.05 101.6) (size 0.8) (drill 0.4) (layers "F.Cu" "B.Cu") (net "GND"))
 (segment (start 161.75 97.75) (end 167.5 97.75) (width 0.75) (layer "F.Cu") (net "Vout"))
 (segment (start 157.675 93.675) (end 161.75 97.75) (width 0.75) (layer "F.Cu") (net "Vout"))
 (segment (start 153.1 102.25) (end 153.1 96.1) (width 0.75) (layer "F.Cu") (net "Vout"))
 (segment (start 153.1 96.1) (end 153.8 95.4) (width 0.75) (layer "F.Cu") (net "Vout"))
 (segment (start 154.325 95.4) (end 156.05 93.675) (width 0.75) (layer "F.Cu") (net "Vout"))
 (segment (start 153.8 95.4) (end 154.325 95.4) (width 0.75) (layer "F.Cu") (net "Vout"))
 (segment (start 156.05 93.675) (end 157.675 93.675) (width 0.75) (layer "F.Cu") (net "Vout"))
 (segment (start 153.8 92.75) (end 153.8 93.75) (width 0.75) (layer "F.Cu") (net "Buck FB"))
 (segment (start 154.8 91.75) (end 153.8 92.75) (width 0.75) (layer "F.Cu") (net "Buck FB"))
 (segment (start 151.4375 93.9125) (end 153.6375 93.9125) (width 0.75) (layer "F.Cu") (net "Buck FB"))
 (segment (start 153.6375 93.9125) (end 153.8 93.75) (width 0.75) (layer "F.Cu") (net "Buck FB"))
 (segment (start 154.8 91.1) (end 154.8 91.75) (width 0.75) (layer "F.Cu") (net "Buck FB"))
 (segment (start 149.1625 94.8625) (end 147.8375 94.8625) (width 0.75) (layer "F.Cu") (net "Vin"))
 (segment (start 146.5 93.525) (end 146.5 92.85) (width 0.75) (layer "F.Cu") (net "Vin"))
 (segment (start 145.025 95) (end 146.5 93.525) (width 0.75) (layer "F.Cu") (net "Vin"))
 (segment (start 146.5 92.85) (end 147.6 91.75) (width 0.75) (layer "F.Cu") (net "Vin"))
 (segment (start 142 95) (end 145.025 95) (width 0.75) (layer "F.Cu") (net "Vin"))
 (segment (start 147.8375 94.8625) (end 146.5 93.525) (width 0.75) (layer "F.Cu") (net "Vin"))
 (segment (start 149.1625 91.8375) (end 149.25 91.75) (width 0.75) (layer "F.Cu") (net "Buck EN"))
 (segment (start 147.5 90) (end 149.25 91.75) (width 0.75) (layer "F.Cu") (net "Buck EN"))
 (segment (start 149.1625 93.9125) (end 149.1625 91.8375) (width 0.75) (layer "F.Cu") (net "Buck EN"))
 (segment (start 151.4375 95.8125) (end 151.4375 97.7125) (width 0.75) (layer "F.Cu") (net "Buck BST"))
 (segment (start 151.4375 97.7125) (end 151.15 98) (width 0.75) (layer "F.Cu") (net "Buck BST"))
 (segment (start 149.25 98) (end 148.4 98) (width 0.75) (layer "F.Cu") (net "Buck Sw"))
 (segment (start 146.4 100) (end 147.15 100) (width 0.75) (layer "F.Cu") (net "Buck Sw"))
 (segment (start 149.1625 97.9125) (end 149.25 98) (width 0.75) (layer "F.Cu") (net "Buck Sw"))
 (segment (start 148.4 98) (end 146.4 100) (width 0.75) (layer "F.Cu") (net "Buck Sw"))
 (segment (start 147.15 100) (end 149.4 102.25) (width 0.75) (layer "F.Cu") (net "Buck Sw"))
 (segment (start 149.1625 95.8125) (end 149.1625 97.9125) (width 0.75) (layer "F.Cu") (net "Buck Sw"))
 (segment (start 152.4 90.35) (end 151 90.35) (width 0.75) (layer "F.Cu") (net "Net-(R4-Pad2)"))
 (segment (start 153.15 91.1) (end 152.4 90.35) (width 0.75) (layer "F.Cu") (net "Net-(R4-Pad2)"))
 (segment (start 133 93.25) (end 140.925 93.25) (width 0.75) (layer "F.Cu") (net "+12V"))
 (segment (start 140.925 93.25) (end 141.05 93.125) (width 0.75) (layer "F.Cu") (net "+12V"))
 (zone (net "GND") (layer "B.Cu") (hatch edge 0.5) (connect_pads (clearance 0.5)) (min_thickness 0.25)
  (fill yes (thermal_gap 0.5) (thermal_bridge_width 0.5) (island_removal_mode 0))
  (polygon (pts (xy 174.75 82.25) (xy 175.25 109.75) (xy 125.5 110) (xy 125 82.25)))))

